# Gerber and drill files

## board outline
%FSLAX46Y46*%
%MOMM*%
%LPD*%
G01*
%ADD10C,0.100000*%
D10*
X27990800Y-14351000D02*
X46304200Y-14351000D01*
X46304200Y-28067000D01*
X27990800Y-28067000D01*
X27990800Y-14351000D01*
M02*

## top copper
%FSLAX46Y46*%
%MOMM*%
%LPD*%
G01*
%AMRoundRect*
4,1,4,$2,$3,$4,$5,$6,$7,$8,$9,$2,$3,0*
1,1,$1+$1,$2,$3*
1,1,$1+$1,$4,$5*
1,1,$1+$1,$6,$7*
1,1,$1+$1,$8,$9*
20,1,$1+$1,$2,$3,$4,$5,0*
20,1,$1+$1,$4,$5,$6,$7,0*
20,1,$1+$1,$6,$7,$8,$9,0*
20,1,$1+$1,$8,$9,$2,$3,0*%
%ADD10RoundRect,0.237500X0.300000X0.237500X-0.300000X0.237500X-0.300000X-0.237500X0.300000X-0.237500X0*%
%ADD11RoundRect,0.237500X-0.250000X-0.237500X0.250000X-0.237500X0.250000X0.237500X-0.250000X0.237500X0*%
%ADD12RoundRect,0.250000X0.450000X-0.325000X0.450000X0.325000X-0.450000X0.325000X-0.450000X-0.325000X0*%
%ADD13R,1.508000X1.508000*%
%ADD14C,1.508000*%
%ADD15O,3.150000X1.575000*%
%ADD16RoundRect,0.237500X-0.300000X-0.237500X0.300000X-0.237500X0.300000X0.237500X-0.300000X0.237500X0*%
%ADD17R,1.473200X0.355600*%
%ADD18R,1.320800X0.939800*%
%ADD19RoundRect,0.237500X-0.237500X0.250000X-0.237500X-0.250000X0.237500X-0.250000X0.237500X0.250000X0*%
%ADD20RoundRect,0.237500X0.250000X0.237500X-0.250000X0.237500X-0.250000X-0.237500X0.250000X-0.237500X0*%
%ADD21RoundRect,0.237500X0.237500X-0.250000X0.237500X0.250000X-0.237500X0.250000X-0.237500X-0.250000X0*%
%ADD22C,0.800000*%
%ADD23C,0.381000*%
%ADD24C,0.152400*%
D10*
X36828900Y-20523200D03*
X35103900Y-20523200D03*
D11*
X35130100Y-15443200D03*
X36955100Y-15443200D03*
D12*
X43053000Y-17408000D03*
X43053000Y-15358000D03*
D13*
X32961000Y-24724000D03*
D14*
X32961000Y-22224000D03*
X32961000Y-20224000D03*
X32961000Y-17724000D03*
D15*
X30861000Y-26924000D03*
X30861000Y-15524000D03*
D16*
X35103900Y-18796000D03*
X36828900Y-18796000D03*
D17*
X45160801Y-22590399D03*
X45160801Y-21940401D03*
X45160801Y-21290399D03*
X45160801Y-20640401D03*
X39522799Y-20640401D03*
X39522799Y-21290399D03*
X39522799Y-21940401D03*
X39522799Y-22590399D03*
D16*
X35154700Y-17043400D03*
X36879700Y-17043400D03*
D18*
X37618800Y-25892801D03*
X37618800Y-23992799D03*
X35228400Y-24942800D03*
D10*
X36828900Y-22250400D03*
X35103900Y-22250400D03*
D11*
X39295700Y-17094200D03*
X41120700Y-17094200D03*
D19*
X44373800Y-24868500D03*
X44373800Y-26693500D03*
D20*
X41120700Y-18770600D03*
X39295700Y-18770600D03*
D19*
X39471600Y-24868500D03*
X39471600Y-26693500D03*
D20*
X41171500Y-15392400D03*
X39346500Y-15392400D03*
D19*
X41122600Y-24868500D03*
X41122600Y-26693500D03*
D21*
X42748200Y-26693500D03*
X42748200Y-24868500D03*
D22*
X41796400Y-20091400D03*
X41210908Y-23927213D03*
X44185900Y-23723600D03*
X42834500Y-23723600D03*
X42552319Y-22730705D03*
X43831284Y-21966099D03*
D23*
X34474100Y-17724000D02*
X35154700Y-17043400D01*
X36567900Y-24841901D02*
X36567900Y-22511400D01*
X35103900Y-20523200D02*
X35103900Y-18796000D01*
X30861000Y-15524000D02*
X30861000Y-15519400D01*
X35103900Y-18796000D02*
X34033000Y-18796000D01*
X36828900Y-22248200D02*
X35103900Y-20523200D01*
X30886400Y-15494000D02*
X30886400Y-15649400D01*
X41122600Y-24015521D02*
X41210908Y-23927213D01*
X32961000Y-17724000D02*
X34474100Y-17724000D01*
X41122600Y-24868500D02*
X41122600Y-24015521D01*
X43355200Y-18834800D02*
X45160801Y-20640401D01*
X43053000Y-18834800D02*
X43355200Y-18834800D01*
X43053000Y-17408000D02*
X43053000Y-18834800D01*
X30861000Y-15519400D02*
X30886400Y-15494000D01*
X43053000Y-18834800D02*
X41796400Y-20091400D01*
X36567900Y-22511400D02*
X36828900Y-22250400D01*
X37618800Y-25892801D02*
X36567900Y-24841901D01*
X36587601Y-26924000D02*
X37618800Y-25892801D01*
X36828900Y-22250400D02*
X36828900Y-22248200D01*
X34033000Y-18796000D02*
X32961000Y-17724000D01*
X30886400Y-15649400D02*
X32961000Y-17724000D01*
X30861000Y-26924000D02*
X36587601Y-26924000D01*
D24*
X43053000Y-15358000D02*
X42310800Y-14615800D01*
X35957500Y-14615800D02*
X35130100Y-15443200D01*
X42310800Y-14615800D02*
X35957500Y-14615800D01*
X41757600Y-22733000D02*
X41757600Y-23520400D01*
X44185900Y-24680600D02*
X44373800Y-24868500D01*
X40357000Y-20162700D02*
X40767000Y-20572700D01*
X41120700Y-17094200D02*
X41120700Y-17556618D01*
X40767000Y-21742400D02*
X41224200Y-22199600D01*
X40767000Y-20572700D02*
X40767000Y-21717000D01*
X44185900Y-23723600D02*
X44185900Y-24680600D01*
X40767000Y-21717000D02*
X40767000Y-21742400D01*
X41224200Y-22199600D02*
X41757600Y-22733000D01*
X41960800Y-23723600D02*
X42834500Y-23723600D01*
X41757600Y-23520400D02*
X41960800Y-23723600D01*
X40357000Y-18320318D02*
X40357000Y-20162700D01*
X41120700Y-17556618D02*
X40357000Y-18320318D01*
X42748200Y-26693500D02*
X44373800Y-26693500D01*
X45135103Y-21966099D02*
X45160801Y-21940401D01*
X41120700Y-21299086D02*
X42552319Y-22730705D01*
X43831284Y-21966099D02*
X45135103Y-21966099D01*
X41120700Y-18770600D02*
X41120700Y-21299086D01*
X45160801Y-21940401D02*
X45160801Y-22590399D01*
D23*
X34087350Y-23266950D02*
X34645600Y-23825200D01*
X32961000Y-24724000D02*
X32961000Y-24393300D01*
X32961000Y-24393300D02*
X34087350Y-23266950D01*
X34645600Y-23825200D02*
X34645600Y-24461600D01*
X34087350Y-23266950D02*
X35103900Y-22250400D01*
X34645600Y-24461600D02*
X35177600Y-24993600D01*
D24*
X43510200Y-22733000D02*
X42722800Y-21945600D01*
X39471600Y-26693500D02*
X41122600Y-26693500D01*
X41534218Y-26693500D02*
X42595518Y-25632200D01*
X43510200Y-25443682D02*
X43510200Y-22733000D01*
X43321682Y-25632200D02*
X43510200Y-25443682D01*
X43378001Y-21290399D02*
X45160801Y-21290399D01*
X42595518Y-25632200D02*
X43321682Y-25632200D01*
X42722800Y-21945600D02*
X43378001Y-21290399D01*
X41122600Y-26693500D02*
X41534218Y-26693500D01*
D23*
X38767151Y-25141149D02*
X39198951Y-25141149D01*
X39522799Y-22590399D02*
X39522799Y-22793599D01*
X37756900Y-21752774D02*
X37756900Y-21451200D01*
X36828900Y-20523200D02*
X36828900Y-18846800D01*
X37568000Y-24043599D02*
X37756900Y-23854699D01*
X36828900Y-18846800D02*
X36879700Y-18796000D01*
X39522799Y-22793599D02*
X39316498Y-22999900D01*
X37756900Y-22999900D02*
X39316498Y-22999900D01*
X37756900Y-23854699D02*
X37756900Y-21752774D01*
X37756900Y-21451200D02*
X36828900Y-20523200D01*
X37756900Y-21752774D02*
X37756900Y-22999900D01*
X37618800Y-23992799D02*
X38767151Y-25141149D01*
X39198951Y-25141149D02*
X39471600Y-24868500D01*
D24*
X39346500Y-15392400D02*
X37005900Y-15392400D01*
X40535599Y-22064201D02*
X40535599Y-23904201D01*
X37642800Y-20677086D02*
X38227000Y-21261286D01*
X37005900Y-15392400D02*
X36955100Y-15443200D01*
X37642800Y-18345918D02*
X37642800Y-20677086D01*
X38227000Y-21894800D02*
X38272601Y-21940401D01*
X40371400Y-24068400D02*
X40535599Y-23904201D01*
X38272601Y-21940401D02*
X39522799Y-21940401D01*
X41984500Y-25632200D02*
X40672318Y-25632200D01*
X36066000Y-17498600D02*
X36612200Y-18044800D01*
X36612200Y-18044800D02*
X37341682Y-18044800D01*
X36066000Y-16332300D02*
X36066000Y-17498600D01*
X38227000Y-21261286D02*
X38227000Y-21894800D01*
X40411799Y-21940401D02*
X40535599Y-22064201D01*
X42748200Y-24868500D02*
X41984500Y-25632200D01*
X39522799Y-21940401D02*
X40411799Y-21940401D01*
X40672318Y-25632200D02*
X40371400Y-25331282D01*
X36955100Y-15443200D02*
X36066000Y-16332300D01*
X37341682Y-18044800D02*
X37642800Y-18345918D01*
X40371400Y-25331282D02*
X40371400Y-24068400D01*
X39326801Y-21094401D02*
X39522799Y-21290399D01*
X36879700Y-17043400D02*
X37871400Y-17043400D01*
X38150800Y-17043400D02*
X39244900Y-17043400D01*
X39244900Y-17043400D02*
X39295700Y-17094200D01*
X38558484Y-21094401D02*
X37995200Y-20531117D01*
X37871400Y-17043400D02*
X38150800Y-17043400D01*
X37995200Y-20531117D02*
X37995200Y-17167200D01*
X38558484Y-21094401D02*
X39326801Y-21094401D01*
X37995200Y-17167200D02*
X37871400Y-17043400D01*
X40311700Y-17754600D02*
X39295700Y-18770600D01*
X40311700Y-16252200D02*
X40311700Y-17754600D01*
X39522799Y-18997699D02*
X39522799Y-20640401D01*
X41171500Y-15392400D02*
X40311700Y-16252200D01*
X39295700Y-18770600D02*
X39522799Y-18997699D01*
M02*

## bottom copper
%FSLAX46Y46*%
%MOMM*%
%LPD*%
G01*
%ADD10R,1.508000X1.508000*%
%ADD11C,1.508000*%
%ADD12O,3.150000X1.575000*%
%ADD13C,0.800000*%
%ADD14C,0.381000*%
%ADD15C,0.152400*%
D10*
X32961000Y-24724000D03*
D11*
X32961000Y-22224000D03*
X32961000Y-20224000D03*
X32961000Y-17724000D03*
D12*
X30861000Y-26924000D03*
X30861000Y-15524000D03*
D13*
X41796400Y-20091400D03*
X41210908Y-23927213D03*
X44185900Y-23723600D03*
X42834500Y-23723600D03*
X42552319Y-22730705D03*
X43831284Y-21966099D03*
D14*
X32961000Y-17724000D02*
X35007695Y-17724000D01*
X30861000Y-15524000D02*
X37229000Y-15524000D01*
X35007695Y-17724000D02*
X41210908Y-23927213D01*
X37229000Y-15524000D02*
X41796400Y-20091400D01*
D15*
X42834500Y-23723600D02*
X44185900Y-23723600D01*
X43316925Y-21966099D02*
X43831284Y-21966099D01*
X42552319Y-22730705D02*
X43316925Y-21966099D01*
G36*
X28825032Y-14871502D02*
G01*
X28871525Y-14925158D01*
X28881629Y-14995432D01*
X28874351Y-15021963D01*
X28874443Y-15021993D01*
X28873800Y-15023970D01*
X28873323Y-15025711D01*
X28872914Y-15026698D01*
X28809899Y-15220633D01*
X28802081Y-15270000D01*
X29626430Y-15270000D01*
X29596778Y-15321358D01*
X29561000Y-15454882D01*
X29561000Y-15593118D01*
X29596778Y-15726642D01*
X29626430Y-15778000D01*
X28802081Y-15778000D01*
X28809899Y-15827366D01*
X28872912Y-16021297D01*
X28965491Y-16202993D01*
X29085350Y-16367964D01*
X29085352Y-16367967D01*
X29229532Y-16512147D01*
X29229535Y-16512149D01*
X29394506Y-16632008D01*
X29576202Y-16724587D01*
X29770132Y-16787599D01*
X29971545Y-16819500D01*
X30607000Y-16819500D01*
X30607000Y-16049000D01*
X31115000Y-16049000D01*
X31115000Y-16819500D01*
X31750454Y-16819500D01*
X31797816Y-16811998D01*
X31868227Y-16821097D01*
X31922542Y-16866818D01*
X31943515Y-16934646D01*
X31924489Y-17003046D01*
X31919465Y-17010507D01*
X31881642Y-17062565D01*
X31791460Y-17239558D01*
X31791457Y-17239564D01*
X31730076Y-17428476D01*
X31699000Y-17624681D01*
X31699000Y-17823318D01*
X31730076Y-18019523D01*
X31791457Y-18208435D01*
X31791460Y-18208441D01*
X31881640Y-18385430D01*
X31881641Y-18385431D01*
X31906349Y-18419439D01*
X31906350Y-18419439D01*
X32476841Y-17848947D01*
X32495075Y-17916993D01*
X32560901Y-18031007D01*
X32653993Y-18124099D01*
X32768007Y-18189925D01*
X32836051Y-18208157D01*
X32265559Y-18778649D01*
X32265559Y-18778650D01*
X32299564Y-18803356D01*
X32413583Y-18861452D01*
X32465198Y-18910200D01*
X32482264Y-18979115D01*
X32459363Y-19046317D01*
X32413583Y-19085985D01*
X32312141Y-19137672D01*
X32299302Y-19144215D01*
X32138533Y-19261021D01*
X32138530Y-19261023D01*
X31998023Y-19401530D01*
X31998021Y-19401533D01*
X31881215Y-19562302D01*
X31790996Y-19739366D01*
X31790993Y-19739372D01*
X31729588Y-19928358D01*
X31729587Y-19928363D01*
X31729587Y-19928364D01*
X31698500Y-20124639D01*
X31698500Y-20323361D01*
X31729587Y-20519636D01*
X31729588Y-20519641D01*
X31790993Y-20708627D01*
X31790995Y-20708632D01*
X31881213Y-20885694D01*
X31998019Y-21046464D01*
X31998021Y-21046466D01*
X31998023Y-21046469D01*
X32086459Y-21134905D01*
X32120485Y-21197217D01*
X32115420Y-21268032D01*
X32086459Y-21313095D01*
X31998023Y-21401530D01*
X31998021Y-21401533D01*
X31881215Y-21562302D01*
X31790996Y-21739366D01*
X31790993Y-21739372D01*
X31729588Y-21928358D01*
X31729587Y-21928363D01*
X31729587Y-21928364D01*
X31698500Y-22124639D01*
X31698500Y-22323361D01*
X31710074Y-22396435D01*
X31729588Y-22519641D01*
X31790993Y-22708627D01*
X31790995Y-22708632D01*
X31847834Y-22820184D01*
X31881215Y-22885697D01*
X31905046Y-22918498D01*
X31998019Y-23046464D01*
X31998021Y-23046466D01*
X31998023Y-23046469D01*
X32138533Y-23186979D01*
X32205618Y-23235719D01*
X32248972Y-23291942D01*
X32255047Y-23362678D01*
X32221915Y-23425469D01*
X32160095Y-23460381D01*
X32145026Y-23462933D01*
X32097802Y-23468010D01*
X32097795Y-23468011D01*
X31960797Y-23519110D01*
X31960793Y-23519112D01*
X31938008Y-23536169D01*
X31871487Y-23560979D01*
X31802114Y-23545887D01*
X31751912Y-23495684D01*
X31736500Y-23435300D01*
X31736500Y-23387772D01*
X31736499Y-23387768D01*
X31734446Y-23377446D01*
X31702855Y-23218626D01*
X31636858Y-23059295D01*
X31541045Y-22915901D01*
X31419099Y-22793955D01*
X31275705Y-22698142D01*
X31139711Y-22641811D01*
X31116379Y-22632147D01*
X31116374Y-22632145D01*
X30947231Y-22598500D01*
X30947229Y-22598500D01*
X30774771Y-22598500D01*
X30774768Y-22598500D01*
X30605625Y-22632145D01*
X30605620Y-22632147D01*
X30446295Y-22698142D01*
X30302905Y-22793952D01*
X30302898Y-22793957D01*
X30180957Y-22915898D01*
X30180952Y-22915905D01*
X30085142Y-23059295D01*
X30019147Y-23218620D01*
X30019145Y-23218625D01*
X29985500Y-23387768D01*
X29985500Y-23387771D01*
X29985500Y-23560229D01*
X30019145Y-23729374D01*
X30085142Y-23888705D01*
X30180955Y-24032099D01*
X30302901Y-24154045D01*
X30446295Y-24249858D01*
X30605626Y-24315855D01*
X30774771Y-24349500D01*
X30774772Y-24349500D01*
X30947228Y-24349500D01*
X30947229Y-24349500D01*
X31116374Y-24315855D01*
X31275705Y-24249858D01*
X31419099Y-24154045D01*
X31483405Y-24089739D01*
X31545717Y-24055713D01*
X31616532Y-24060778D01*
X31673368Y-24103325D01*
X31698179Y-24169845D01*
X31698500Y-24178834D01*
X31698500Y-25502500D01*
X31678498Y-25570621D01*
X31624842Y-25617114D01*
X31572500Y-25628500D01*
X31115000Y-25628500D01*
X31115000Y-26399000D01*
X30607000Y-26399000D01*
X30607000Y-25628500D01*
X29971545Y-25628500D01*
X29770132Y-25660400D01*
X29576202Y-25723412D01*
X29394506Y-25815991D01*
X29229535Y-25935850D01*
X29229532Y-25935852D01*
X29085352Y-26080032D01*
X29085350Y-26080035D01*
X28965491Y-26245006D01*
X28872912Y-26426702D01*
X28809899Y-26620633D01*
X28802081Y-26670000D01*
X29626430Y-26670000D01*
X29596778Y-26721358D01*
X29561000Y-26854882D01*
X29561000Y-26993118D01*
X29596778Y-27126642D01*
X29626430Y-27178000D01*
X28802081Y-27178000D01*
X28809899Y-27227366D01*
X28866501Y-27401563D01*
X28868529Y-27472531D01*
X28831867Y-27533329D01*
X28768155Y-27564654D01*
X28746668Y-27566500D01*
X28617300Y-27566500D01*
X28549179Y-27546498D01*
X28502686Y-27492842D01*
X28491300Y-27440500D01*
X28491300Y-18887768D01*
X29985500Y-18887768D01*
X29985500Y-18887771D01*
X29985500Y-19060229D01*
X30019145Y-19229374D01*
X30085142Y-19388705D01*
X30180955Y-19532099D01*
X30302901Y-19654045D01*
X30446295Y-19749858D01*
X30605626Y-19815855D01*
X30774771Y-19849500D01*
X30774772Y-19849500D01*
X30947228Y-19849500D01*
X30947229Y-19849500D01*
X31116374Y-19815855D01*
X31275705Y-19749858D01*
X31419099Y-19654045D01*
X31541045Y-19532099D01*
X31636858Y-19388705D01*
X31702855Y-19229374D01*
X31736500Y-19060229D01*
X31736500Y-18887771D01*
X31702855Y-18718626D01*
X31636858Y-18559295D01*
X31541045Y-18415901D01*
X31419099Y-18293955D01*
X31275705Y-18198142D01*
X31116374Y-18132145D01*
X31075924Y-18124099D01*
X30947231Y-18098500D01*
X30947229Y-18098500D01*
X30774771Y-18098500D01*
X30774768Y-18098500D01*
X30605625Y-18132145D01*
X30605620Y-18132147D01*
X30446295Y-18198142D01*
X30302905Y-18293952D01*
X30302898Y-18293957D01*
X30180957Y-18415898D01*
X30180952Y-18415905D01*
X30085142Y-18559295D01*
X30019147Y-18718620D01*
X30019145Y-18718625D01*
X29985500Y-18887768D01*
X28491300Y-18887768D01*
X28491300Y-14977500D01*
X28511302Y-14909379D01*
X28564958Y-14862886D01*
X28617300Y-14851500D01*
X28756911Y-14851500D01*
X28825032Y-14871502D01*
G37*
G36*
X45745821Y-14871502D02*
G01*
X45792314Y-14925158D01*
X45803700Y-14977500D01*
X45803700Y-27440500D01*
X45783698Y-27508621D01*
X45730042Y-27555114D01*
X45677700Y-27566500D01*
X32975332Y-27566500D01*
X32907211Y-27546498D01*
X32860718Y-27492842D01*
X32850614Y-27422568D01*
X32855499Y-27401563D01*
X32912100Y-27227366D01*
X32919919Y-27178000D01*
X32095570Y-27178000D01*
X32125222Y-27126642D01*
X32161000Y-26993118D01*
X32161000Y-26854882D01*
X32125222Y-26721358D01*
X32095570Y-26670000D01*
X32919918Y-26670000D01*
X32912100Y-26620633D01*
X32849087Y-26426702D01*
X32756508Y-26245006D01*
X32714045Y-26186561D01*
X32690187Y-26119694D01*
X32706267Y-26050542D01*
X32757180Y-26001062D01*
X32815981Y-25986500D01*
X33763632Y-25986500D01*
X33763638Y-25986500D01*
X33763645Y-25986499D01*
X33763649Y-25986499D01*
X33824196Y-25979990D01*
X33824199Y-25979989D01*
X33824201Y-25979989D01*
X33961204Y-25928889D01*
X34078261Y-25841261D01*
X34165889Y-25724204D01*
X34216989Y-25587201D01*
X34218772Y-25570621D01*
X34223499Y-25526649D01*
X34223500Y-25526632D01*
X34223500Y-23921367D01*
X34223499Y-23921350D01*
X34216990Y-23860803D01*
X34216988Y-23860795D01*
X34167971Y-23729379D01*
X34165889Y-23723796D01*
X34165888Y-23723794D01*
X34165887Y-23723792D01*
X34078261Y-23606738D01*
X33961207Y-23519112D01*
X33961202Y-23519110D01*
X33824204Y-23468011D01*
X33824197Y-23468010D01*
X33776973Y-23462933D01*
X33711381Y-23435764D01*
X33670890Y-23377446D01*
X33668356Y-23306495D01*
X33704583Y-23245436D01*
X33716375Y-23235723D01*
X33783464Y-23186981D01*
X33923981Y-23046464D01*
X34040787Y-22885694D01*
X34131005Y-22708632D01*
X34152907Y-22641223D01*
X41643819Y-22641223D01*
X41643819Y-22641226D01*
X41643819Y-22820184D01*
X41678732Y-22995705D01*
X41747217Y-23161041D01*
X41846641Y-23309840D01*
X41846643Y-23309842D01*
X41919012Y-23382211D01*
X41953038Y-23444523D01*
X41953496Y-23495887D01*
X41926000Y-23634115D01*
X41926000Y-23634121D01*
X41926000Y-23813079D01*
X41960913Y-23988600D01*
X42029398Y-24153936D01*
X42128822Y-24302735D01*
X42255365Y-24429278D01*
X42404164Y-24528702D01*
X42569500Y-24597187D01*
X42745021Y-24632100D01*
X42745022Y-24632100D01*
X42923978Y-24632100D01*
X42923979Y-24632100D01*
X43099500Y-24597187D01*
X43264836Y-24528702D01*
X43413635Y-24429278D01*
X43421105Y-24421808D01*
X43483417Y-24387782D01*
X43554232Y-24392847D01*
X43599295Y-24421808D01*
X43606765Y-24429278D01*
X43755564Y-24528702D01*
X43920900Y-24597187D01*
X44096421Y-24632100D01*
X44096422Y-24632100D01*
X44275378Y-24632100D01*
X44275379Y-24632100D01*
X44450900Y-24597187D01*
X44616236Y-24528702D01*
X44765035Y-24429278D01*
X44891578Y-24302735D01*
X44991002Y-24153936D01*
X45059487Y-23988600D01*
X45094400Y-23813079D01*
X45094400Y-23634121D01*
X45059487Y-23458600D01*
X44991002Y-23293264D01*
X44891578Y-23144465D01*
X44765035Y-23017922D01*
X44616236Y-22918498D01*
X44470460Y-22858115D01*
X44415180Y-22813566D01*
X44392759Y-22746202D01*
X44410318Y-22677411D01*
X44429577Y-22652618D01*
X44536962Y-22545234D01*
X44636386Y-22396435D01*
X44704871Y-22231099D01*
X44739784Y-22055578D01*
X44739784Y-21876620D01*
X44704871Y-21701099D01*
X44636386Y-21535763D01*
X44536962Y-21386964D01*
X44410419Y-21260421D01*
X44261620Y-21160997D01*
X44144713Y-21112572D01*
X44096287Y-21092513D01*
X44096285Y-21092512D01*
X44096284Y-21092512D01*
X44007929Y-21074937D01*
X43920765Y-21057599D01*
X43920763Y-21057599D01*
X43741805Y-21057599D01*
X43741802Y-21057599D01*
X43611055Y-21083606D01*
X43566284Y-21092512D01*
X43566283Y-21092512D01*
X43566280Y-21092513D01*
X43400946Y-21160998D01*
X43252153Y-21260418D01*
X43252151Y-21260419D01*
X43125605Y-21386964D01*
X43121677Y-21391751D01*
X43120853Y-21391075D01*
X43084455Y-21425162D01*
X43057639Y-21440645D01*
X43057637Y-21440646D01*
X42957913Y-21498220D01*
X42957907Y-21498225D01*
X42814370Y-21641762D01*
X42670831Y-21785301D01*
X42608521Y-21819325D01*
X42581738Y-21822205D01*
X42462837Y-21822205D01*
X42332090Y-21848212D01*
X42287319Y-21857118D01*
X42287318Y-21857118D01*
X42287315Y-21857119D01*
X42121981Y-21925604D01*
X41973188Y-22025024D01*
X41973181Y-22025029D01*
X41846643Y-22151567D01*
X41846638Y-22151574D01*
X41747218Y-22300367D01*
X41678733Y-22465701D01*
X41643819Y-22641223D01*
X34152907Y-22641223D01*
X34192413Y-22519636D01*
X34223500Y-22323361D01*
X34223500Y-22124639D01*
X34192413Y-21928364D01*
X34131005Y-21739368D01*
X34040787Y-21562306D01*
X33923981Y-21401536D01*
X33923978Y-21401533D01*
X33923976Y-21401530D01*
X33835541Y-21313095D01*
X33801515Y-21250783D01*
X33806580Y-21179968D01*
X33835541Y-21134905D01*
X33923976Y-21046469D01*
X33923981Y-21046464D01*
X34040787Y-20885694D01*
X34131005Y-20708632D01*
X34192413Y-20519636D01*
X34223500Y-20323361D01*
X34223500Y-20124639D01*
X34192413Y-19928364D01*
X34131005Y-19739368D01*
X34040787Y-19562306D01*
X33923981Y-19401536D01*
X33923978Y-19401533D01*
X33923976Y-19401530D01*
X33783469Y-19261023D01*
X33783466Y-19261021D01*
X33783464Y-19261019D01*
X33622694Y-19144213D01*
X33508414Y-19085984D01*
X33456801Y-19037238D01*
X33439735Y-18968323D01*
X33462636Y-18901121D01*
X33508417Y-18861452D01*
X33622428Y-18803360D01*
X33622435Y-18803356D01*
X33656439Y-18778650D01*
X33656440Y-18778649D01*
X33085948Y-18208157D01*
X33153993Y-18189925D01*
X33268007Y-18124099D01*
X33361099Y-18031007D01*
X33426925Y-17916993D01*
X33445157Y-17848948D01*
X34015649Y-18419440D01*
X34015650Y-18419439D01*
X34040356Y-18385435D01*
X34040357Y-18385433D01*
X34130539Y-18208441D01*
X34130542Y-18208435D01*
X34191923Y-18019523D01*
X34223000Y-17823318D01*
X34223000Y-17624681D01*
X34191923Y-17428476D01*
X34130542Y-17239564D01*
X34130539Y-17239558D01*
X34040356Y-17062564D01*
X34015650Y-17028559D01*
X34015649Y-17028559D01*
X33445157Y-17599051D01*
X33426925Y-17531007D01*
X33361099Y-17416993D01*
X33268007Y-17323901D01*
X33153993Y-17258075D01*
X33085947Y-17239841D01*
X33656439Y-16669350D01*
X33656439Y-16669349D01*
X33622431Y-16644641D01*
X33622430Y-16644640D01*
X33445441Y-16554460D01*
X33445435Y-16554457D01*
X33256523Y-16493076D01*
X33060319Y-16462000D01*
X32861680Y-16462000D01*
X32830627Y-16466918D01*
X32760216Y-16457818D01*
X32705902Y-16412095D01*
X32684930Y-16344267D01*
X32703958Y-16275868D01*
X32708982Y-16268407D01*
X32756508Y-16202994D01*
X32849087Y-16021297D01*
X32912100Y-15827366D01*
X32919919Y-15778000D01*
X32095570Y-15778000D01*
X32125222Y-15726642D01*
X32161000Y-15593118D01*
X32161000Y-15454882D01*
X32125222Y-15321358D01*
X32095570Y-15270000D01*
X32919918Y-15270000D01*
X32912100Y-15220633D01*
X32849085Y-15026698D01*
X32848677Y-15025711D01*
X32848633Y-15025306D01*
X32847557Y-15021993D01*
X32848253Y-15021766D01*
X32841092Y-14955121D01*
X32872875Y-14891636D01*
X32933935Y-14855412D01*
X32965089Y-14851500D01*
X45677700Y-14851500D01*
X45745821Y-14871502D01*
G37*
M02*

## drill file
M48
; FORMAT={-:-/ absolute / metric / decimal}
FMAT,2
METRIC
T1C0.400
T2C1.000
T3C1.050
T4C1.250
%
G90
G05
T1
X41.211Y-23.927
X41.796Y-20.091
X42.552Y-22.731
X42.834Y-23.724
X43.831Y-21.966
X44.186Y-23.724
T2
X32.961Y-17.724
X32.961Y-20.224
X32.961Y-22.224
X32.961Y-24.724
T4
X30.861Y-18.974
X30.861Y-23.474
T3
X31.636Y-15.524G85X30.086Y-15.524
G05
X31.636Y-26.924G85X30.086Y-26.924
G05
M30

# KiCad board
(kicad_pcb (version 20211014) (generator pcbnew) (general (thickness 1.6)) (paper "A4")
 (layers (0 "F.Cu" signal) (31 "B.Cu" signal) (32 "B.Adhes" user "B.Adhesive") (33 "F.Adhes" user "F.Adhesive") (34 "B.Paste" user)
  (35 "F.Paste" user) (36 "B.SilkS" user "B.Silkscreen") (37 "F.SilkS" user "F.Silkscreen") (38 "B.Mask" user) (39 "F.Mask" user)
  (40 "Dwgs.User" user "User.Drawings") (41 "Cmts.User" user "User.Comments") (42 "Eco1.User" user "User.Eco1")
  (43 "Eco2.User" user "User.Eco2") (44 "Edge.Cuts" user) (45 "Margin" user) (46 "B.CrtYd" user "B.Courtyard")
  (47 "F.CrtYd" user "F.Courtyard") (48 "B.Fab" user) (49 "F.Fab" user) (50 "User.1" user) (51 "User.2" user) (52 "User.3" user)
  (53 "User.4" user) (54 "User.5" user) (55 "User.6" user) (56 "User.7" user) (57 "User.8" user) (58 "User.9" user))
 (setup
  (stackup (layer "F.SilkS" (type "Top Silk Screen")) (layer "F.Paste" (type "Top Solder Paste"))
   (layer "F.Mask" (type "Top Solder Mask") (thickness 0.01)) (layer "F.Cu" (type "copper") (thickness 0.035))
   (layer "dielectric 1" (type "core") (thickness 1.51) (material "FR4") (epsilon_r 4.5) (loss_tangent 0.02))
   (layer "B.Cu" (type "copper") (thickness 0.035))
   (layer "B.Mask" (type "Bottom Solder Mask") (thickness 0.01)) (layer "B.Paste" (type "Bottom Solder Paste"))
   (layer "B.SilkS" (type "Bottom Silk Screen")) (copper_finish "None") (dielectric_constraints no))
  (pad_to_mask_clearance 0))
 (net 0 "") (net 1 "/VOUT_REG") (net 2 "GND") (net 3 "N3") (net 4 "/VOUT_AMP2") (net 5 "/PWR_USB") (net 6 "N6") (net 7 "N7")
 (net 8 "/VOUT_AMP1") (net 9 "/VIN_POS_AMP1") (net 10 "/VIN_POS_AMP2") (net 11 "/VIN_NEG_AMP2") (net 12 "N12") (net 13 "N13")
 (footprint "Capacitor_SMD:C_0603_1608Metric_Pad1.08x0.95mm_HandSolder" (layer "F.Cu") (at 35.9664 20.5232 180)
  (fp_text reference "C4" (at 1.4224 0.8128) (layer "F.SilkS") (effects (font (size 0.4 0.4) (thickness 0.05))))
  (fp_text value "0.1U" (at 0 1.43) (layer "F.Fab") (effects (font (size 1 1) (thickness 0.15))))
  (pad "1" smd roundrect (at -0.8625 0 180) (size 1.075 0.95) (layers "F.Cu" "F.Paste" "F.Mask") (roundrect_rratio 0.25) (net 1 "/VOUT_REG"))
  (pad "2" smd roundrect (at 0.8625 0 180) (size 1.075 0.95) (layers "F.Cu" "F.Paste" "F.Mask") (roundrect_rratio 0.25) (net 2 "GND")))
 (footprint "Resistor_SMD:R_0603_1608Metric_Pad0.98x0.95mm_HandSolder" (layer "F.Cu") (at 36.0426 15.4432)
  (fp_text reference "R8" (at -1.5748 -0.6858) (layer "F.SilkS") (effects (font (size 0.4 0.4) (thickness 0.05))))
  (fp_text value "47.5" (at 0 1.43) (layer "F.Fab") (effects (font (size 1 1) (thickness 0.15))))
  (pad "1" smd roundrect (at -0.9125 0) (size 0.975 0.95) (layers "F.Cu" "F.Paste" "F.Mask") (roundrect_rratio 0.25) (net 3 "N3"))
  (pad "2" smd roundrect (at 0.9125 0) (size 0.975 0.95) (layers "F.Cu" "F.Paste" "F.Mask") (roundrect_rratio 0.25) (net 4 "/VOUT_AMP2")))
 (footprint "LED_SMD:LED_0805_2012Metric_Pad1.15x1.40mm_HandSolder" (layer "F.Cu") (at 43.053 16.383 90)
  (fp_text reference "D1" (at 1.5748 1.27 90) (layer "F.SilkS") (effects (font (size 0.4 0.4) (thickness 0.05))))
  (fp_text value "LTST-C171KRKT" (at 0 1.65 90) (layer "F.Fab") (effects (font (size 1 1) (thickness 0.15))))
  (pad "1" smd roundrect (at -1.025 0 90) (size 1.15 1.4) (layers "F.Cu" "F.Paste" "F.Mask") (roundrect_rratio 0.217391) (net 2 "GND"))
  (pad "2" smd roundrect (at 1.025 0 90) (size 1.15 1.4) (layers "F.Cu" "F.Paste" "F.Mask") (roundrect_rratio 0.217391) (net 3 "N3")))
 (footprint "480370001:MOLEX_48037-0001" (layer "F.Cu") (at 30.861 21.224 -90)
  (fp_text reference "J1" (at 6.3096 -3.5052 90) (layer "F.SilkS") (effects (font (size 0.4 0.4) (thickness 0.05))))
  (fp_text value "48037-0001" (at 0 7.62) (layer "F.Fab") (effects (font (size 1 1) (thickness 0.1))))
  (pad "" np_thru_hole circle (at -2.25 0 270) (size 1.25 1.25) (drill 1.25) (layers *.Cu *.Mask))
  (pad "" np_thru_hole circle (at 2.25 0 270) (size 1.25 1.25) (drill 1.25) (layers *.Cu *.Mask))
  (pad "1" thru_hole rect (at 3.5 -2.1 270) (size 1.508 1.508) (drill 1) (layers *.Cu *.Mask) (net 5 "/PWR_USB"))
  (pad "2" thru_hole circle (at 1 -2.1 270) (size 1.508 1.508) (drill 1) (layers *.Cu *.Mask) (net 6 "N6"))
  (pad "3" thru_hole circle (at -1 -2.1 270) (size 1.508 1.508) (drill 1) (layers *.Cu *.Mask) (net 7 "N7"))
  (pad "4" thru_hole circle (at -3.5 -2.1 270) (size 1.508 1.508) (drill 1) (layers *.Cu *.Mask) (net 2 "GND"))
  (pad "S1" thru_hole oval (at 5.7 0 270) (size 1.575 3.15) (drill oval 1.05 2.6) (layers *.Cu *.Mask) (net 2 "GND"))
  (pad "S2" thru_hole oval (at -5.7 0 270) (size 1.575 3.15) (drill oval 1.05 2.6) (layers *.Cu *.Mask) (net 2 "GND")))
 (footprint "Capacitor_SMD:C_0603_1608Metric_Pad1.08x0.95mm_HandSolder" (layer "F.Cu") (at 35.9664 18.796)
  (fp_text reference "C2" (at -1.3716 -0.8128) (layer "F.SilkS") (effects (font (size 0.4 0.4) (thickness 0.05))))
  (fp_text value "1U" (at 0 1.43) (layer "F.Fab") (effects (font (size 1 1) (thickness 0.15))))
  (pad "1" smd roundrect (at -0.8625 0) (size 1.075 0.95) (layers "F.Cu" "F.Paste" "F.Mask") (roundrect_rratio 0.25) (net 2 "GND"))
  (pad "2" smd roundrect (at 0.8625 0) (size 1.075 0.95) (layers "F.Cu" "F.Paste" "F.Mask") (roundrect_rratio 0.25) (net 1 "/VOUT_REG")))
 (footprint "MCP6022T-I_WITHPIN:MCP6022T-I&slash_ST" (layer "F.Cu") (at 42.3418 21.6154 180)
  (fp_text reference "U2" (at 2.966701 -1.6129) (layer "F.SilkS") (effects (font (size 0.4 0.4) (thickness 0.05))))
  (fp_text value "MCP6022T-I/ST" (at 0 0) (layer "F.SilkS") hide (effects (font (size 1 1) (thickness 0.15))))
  (pad "1" smd rect (at -2.819001 -0.974999 180) (size 1.4732 0.3556) (layers "F.Cu" "F.Paste" "F.Mask") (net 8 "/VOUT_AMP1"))
  (pad "2" smd rect (at -2.819001 -0.325001 180) (size 1.4732 0.3556) (layers "F.Cu" "F.Paste" "F.Mask") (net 8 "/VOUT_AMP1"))
  (pad "3" smd rect (at -2.819001 0.325001 180) (size 1.4732 0.3556) (layers "F.Cu" "F.Paste" "F.Mask") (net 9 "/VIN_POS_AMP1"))
  (pad "4" smd rect (at -2.819001 0.974999 180) (size 1.4732 0.3556) (layers "F.Cu" "F.Paste" "F.Mask") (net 2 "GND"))
  (pad "5" smd rect (at 2.819001 0.974999 180) (size 1.4732 0.3556) (layers "F.Cu" "F.Paste" "F.Mask") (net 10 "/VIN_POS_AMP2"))
  (pad "6" smd rect (at 2.819001 0.325001 180) (size 1.4732 0.3556) (layers "F.Cu" "F.Paste" "F.Mask") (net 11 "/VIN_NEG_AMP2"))
  (pad "7" smd rect (at 2.819001 -0.325001 180) (size 1.4732 0.3556) (layers "F.Cu" "F.Paste" "F.Mask") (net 4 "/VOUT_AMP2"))
  (pad "8" smd rect (at 2.819001 -0.974999 180) (size 1.4732 0.3556) (layers "F.Cu" "F.Paste" "F.Mask") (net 1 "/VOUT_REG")))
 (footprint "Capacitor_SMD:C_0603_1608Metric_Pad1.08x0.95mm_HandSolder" (layer "F.Cu") (at 36.0172 17.0434)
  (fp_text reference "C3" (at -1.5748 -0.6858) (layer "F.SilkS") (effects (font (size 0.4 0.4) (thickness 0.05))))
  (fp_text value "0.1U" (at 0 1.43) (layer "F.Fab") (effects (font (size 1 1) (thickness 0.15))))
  (pad "1" smd roundrect (at -0.8625 0) (size 1.075 0.95) (layers "F.Cu" "F.Paste" "F.Mask") (roundrect_rratio 0.25) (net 2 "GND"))
  (pad "2" smd roundrect (at 0.8625 0) (size 1.075 0.95) (layers "F.Cu" "F.Paste" "F.Mask") (roundrect_rratio 0.25) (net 11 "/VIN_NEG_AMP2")))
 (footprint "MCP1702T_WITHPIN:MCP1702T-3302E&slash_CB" (layer "F.Cu") (at 36.4236 24.9428 90)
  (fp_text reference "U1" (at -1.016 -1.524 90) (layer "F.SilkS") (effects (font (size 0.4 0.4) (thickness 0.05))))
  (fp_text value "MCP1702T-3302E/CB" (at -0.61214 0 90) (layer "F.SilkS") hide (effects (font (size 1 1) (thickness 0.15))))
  (pad "1" smd rect (at -0.950001 1.1952 90) (size 0.9398 1.3208) (layers "F.Cu" "F.Paste" "F.Mask") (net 2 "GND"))
  (pad "2" smd rect (at 0.950001 1.1952 90) (size 0.9398 1.3208) (layers "F.Cu" "F.Paste" "F.Mask") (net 1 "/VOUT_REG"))
  (pad "3" smd rect (at 0 -1.1952 90) (size 0.9398 1.3208) (layers "F.Cu" "F.Paste" "F.Mask") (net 5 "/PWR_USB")))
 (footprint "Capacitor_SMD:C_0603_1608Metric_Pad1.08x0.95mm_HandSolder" (layer "F.Cu") (at 35.9664 22.2504 180)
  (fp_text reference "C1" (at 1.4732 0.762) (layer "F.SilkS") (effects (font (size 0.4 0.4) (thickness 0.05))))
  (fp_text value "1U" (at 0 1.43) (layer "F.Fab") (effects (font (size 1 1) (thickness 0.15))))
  (pad "1" smd roundrect (at -0.8625 0 180) (size 1.075 0.95) (layers "F.Cu" "F.Paste" "F.Mask") (roundrect_rratio 0.25) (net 2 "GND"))
  (pad "2" smd roundrect (at 0.8625 0 180) (size 1.075 0.95) (layers "F.Cu" "F.Paste" "F.Mask") (roundrect_rratio 0.25) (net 5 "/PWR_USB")))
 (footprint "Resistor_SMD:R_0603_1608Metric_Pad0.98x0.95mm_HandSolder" (layer "F.Cu") (at 40.2082 17.0942)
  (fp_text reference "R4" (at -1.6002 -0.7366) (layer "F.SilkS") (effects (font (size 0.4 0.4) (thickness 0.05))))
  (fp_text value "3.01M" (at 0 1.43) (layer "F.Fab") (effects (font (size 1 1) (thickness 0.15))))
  (pad "1" smd roundrect (at -0.9125 0) (size 0.975 0.95) (layers "F.Cu" "F.Paste" "F.Mask") (roundrect_rratio 0.25)
   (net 11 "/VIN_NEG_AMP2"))
  (pad "2" smd roundrect (at 0.9125 0) (size 0.975 0.95) (layers "F.Cu" "F.Paste" "F.Mask") (roundrect_rratio 0.25) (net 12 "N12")))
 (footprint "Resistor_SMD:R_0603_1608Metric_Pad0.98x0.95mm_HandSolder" (layer "F.Cu") (at 44.3738 25.781 -90)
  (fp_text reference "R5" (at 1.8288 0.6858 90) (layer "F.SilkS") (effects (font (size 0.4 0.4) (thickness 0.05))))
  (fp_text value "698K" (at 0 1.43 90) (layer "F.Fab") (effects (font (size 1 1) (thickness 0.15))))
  (pad "1" smd roundrect (at -0.9125 0 270) (size 0.975 0.95) (layers "F.Cu" "F.Paste" "F.Mask") (roundrect_rratio 0.25) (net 12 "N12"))
  (pad "2" smd roundrect (at 0.9125 0 270) (size 0.975 0.95) (layers "F.Cu" "F.Paste" "F.Mask") (roundrect_rratio 0.25) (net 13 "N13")))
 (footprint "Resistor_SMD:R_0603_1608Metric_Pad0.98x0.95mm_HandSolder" (layer "F.Cu") (at 40.2082 18.7706 180)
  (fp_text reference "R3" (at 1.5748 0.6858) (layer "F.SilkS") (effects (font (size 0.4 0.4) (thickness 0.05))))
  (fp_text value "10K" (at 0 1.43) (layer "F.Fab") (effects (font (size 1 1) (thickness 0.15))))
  (pad "1" smd roundrect (at -0.9125 0 180) (size 0.975 0.95) (layers "F.Cu" "F.Paste" "F.Mask") (roundrect_rratio 0.25)
   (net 8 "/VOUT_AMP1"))
  (pad "2" smd roundrect (at 0.9125 0 180) (size 0.975 0.95) (layers "F.Cu" "F.Paste" "F.Mask") (roundrect_rratio 0.25)
   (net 10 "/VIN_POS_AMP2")))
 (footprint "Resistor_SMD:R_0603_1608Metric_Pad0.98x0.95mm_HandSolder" (layer "F.Cu") (at 39.4716 25.781 -90)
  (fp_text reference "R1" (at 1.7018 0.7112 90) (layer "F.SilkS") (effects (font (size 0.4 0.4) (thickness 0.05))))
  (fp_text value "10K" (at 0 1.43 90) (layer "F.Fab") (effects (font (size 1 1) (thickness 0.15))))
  (pad "1" smd roundrect (at -0.9125 0 270) (size 0.975 0.95) (layers "F.Cu" "F.Paste" "F.Mask") (roundrect_rratio 0.25) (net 1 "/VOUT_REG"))
  (pad "2" smd roundrect (at 0.9125 0 270) (size 0.975 0.95) (layers "F.Cu" "F.Paste" "F.Mask") (roundrect_rratio 0.25)
   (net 9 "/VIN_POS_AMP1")))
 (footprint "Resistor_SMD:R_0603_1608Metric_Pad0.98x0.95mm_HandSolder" (layer "F.Cu") (at 40.259 15.3924 180)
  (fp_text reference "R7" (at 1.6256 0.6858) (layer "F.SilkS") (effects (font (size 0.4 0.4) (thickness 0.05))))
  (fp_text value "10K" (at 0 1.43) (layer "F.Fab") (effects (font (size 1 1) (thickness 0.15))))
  (pad "1" smd roundrect (at -0.9125 0 180) (size 0.975 0.95) (layers "F.Cu" "F.Paste" "F.Mask") (roundrect_rratio 0.25)
   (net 10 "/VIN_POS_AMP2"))
  (pad "2" smd roundrect (at 0.9125 0 180) (size 0.975 0.95) (layers "F.Cu" "F.Paste" "F.Mask") (roundrect_rratio 0.25) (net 4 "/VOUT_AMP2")))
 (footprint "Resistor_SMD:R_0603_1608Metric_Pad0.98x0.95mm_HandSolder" (layer "F.Cu") (at 41.1226 25.781 -90)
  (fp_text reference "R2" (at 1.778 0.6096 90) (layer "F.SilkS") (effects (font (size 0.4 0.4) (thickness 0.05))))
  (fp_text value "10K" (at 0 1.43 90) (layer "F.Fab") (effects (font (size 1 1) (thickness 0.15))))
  (pad "1" smd roundrect (at -0.9125 0 270) (size 0.975 0.95) (layers "F.Cu" "F.Paste" "F.Mask") (roundrect_rratio 0.25) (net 2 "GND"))
  (pad "2" smd roundrect (at 0.9125 0 270) (size 0.975 0.95) (layers "F.Cu" "F.Paste" "F.Mask") (roundrect_rratio 0.25)
   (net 9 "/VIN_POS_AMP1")))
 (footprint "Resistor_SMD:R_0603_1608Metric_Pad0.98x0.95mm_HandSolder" (layer "F.Cu") (at 42.7482 25.781 90)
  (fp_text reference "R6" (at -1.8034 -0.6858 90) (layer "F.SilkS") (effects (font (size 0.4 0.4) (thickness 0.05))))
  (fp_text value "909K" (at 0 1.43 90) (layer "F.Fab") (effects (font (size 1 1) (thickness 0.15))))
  (pad "1" smd roundrect (at -0.9125 0 90) (size 0.975 0.95) (layers "F.Cu" "F.Paste" "F.Mask") (roundrect_rratio 0.25) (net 13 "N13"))
  (pad "2" smd roundrect (at 0.9125 0 90) (size 0.975 0.95) (layers "F.Cu" "F.Paste" "F.Mask") (roundrect_rratio 0.25) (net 4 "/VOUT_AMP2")))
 (gr_rect (start 46.3042 28.067) (end 27.9908 14.351) (layer "Edge.Cuts") (width 0.1) (fill none))
 (segment (start 34.4741 17.724) (end 35.1547 17.0434) (width 0.381) (layer "F.Cu") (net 2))
 (segment (start 36.5679 24.841901) (end 36.5679 22.5114) (width 0.381) (layer "F.Cu") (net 2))
 (segment (start 35.1039 20.5232) (end 35.1039 18.796) (width 0.381) (layer "F.Cu") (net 2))
 (segment (start 30.861 15.524) (end 30.861 15.5194) (width 0.381) (layer "F.Cu") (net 2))
 (segment (start 35.1039 18.796) (end 34.033 18.796) (width 0.381) (layer "F.Cu") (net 2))
 (segment (start 36.8289 22.2482) (end 35.1039 20.5232) (width 0.381) (layer "F.Cu") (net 2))
 (segment (start 30.8864 15.494) (end 30.8864 15.6494) (width 0.381) (layer "F.Cu") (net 2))
 (segment (start 41.1226 24.015521) (end 41.210908 23.927213) (width 0.381) (layer "F.Cu") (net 2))
 (segment (start 32.961 17.724) (end 34.4741 17.724) (width 0.381) (layer "F.Cu") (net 2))
 (segment (start 41.1226 24.8685) (end 41.1226 24.015521) (width 0.381) (layer "F.Cu") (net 2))
 (segment (start 43.3552 18.8348) (end 45.160801 20.640401) (width 0.381) (layer "F.Cu") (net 2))
 (segment (start 43.053 18.8348) (end 43.3552 18.8348) (width 0.381) (layer "F.Cu") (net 2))
 (segment (start 43.053 17.408) (end 43.053 18.8348) (width 0.381) (layer "F.Cu") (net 2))
 (segment (start 30.861 15.5194) (end 30.8864 15.494) (width 0.381) (layer "F.Cu") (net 2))
 (segment (start 43.053 18.8348) (end 41.7964 20.0914) (width 0.381) (layer "F.Cu") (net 2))
 (segment (start 36.5679 22.5114) (end 36.8289 22.2504) (width 0.381) (layer "F.Cu") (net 2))
 (segment (start 37.6188 25.892801) (end 36.5679 24.841901) (width 0.381) (layer "F.Cu") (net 2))
 (segment (start 36.587601 26.924) (end 37.6188 25.892801) (width 0.381) (layer "F.Cu") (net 2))
 (segment (start 36.8289 22.2504) (end 36.8289 22.2482) (width 0.381) (layer "F.Cu") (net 2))
 (segment (start 34.033 18.796) (end 32.961 17.724) (width 0.381) (layer "F.Cu") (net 2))
 (segment (start 30.8864 15.6494) (end 32.961 17.724) (width 0.381) (layer "F.Cu") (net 2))
 (segment (start 30.861 26.924) (end 36.587601 26.924) (width 0.381) (layer "F.Cu") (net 2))
 (via (at 41.7964 20.0914) (size 0.8) (drill 0.4) (layers "F.Cu" "B.Cu") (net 2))
 (via (at 41.210908 23.927213) (size 0.8) (drill 0.4) (layers "F.Cu" "B.Cu") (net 2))
 (segment (start 32.961 17.724) (end 35.007695 17.724) (width 0.381) (layer "B.Cu") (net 2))
 (segment (start 30.861 15.524) (end 37.229 15.524) (width 0.381) (layer "B.Cu") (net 2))
 (segment (start 35.007695 17.724) (end 41.210908 23.927213) (width 0.381) (layer "B.Cu") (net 2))
 (segment (start 37.229 15.524) (end 41.7964 20.0914) (width 0.381) (layer "B.Cu") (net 2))
 (segment (start 43.053 15.358) (end 42.3108 14.6158) (width 0.1524) (layer "F.Cu") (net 3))
 (segment (start 35.9575 14.6158) (end 35.1301 15.4432) (width 0.1524) (layer "F.Cu") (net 3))
 (segment (start 42.3108 14.6158) (end 35.9575 14.6158) (width 0.1524) (layer "F.Cu") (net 3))
 (segment (start 41.7576 22.733) (end 41.7576 23.5204) (width 0.1524) (layer "F.Cu") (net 12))
 (segment (start 44.1859 24.6806) (end 44.3738 24.8685) (width 0.1524) (layer "F.Cu") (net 12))
 (segment (start 40.357 20.1627) (end 40.767 20.5727) (width 0.1524) (layer "F.Cu") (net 12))
 (segment (start 41.1207 17.0942) (end 41.1207 17.556618) (width 0.1524) (layer "F.Cu") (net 12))
 (segment (start 40.767 21.7424) (end 41.2242 22.1996) (width 0.1524) (layer "F.Cu") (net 12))
 (segment (start 40.767 20.5727) (end 40.767 21.717) (width 0.1524) (layer "F.Cu") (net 12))
 (segment (start 44.1859 23.7236) (end 44.1859 24.6806) (width 0.1524) (layer "F.Cu") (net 12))
 (segment (start 40.767 21.717) (end 40.767 21.7424) (width 0.1524) (layer "F.Cu") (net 12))
 (segment (start 41.2242 22.1996) (end 41.7576 22.733) (width 0.1524) (layer "F.Cu") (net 12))
 (segment (start 41.9608 23.7236) (end 42.8345 23.7236) (width 0.1524) (layer "F.Cu") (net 12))
 (segment (start 41.7576 23.5204) (end 41.9608 23.7236) (width 0.1524) (layer "F.Cu") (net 12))
 (segment (start 40.357 18.320318) (end 40.357 20.1627) (width 0.1524) (layer "F.Cu") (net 12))
 (segment (start 41.1207 17.556618) (end 40.357 18.320318) (width 0.1524) (layer "F.Cu") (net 12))
 (via (at 44.1859 23.7236) (size 0.8) (drill 0.4) (layers "F.Cu" "B.Cu") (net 12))
 (via (at 42.8345 23.7236) (size 0.8) (drill 0.4) (layers "F.Cu" "B.Cu") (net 12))
 (segment (start 42.8345 23.7236) (end 44.1859 23.7236) (width 0.1524) (layer "B.Cu") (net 12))
 (segment (start 42.7482 26.6935) (end 44.3738 26.6935) (width 0.1524) (layer "F.Cu") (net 13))
 (segment (start 45.135103 21.966099) (end 45.160801 21.940401) (width 0.1524) (layer "F.Cu") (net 8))
 (segment (start 41.1207 21.299086) (end 42.552319 22.730705) (width 0.1524) (layer "F.Cu") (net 8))
 (segment (start 43.831284 21.966099) (end 45.135103 21.966099) (width 0.1524) (layer "F.Cu") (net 8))
 (segment (start 41.1207 18.7706) (end 41.1207 21.299086) (width 0.1524) (layer "F.Cu") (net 8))
 (segment (start 45.160801 21.940401) (end 45.160801 22.590399) (width 0.1524) (layer "F.Cu") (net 8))
 (via (at 42.552319 22.730705) (size 0.8) (drill 0.4) (layers "F.Cu" "B.Cu") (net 8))
 (via (at 43.831284 21.966099) (size 0.8) (drill 0.4) (layers "F.Cu" "B.Cu") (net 8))
 (segment (start 43.316925 21.966099) (end 43.831284 21.966099) (width 0.1524) (layer "B.Cu") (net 8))
 (segment (start 42.552319 22.730705) (end 43.316925 21.966099) (width 0.1524) (layer "B.Cu") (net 8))
 (segment (start 34.08735 23.26695) (end 34.6456 23.8252) (width 0.381) (layer "F.Cu") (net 5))
 (segment (start 32.961 24.724) (end 32.961 24.3933) (width 0.381) (layer "F.Cu") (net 5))
 (segment (start 32.961 24.3933) (end 34.08735 23.26695) (width 0.381) (layer "F.Cu") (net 5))
 (segment (start 34.6456 23.8252) (end 34.6456 24.4616) (width 0.381) (layer "F.Cu") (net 5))
 (segment (start 34.08735 23.26695) (end 35.1039 22.2504) (width 0.381) (layer "F.Cu") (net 5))
 (segment (start 34.6456 24.4616) (end 35.1776 24.9936) (width 0.381) (layer "F.Cu") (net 5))
 (segment (start 43.5102 22.733) (end 42.7228 21.9456) (width 0.1524) (layer "F.Cu") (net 9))
 (segment (start 39.4716 26.6935) (end 41.1226 26.6935) (width 0.1524) (layer "F.Cu") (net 9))
 (segment (start 41.534218 26.6935) (end 42.595518 25.6322) (width 0.1524) (layer "F.Cu") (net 9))
 (segment (start 43.5102 25.443682) (end 43.5102 22.733) (width 0.1524) (layer "F.Cu") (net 9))
 (segment (start 43.321682 25.6322) (end 43.5102 25.443682) (width 0.1524) (layer "F.Cu") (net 9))
 (segment (start 43.378001 21.290399) (end 45.160801 21.290399) (width 0.1524) (layer "F.Cu") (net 9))
 (segment (start 42.595518 25.6322) (end 43.321682 25.6322) (width 0.1524) (layer "F.Cu") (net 9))
 (segment (start 42.7228 21.9456) (end 43.378001 21.290399) (width 0.1524) (layer "F.Cu") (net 9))
 (segment (start 41.1226 26.6935) (end 41.534218 26.6935) (width 0.1524) (layer "F.Cu") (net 9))
 (segment (start 38.767151 25.141149) (end 39.198951 25.141149) (width 0.381) (layer "F.Cu") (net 1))
 (segment (start 39.522799 22.590399) (end 39.522799 22.793599) (width 0.381) (layer "F.Cu") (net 1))
 (segment (start 37.7569 21.752774) (end 37.7569 21.4512) (width 0.381) (layer "F.Cu") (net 1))
 (segment (start 36.8289 20.5232) (end 36.8289 18.8468) (width 0.381) (layer "F.Cu") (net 1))
 (segment (start 37.568 24.043599) (end 37.7569 23.854699) (width 0.381) (layer "F.Cu") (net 1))
 (segment (start 36.8289 18.8468) (end 36.8797 18.796) (width 0.381) (layer "F.Cu") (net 1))
 (segment (start 39.522799 22.793599) (end 39.316498 22.9999) (width 0.381) (layer "F.Cu") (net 1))
 (segment (start 37.7569 22.9999) (end 39.316498 22.9999) (width 0.381) (layer "F.Cu") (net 1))
 (segment (start 37.7569 23.854699) (end 37.7569 21.752774) (width 0.381) (layer "F.Cu") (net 1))
 (segment (start 37.7569 21.4512) (end 36.8289 20.5232) (width 0.381) (layer "F.Cu") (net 1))
 (segment (start 37.7569 21.752774) (end 37.7569 22.9999) (width 0.381) (layer "F.Cu") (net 1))
 (segment (start 37.6188 23.992799) (end 38.767151 25.141149) (width 0.381) (layer "F.Cu") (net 1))
 (segment (start 39.198951 25.141149) (end 39.4716 24.8685) (width 0.381) (layer "F.Cu") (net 1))
 (segment (start 39.3465 15.3924) (end 37.0059 15.3924) (width 0.1524) (layer "F.Cu") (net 4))
 (segment (start 40.535599 22.064201) (end 40.535599 23.904201) (width 0.1524) (layer "F.Cu") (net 4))
 (segment (start 37.6428 20.677086) (end 38.227 21.261286) (width 0.1524) (layer "F.Cu") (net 4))
 (segment (start 37.0059 15.3924) (end 36.9551 15.4432) (width 0.1524) (layer "F.Cu") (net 4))
 (segment (start 37.6428 18.345918) (end 37.6428 20.677086) (width 0.1524) (layer "F.Cu") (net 4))
 (segment (start 38.227 21.8948) (end 38.272601 21.940401) (width 0.1524) (layer "F.Cu") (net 4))
 (segment (start 40.3714 24.0684) (end 40.535599 23.904201) (width 0.1524) (layer "F.Cu") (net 4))
 (segment (start 38.272601 21.940401) (end 39.522799 21.940401) (width 0.1524) (layer "F.Cu") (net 4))
 (segment (start 41.9845 25.6322) (end 40.672318 25.6322) (width 0.1524) (layer "F.Cu") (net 4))
 (segment (start 36.066 17.4986) (end 36.6122 18.0448) (width 0.1524) (layer "F.Cu") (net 4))
 (segment (start 36.6122 18.0448) (end 37.341682 18.0448) (width 0.1524) (layer "F.Cu") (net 4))
 (segment (start 36.066 16.3323) (end 36.066 17.4986) (width 0.1524) (layer "F.Cu") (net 4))
 (segment (start 38.227 21.261286) (end 38.227 21.8948) (width 0.1524) (layer "F.Cu") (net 4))
 (segment (start 40.411799 21.940401) (end 40.535599 22.064201) (width 0.1524) (layer "F.Cu") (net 4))
 (segment (start 42.7482 24.8685) (end 41.9845 25.6322) (width 0.1524) (layer "F.Cu") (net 4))
 (segment (start 39.522799 21.940401) (end 40.411799 21.940401) (width 0.1524) (layer "F.Cu") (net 4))
 (segment (start 40.672318 25.6322) (end 40.3714 25.331282) (width 0.1524) (layer "F.Cu") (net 4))
 (segment (start 36.9551 15.4432) (end 36.066 16.3323) (width 0.1524) (layer "F.Cu") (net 4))
 (segment (start 37.341682 18.0448) (end 37.6428 18.345918) (width 0.1524) (layer "F.Cu") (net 4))
 (segment (start 40.3714 25.331282) (end 40.3714 24.0684) (width 0.1524) (layer "F.Cu") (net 4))
 (segment (start 39.326801 21.094401) (end 39.522799 21.290399) (width 0.1524) (layer "F.Cu") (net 11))
 (segment (start 36.8797 17.0434) (end 37.8714 17.0434) (width 0.1524) (layer "F.Cu") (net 11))
 (segment (start 38.1508 17.0434) (end 39.2449 17.0434) (width 0.1524) (layer "F.Cu") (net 11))
 (segment (start 39.2449 17.0434) (end 39.2957 17.0942) (width 0.1524) (layer "F.Cu") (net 11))
 (segment (start 38.558484 21.094401) (end 37.9952 20.531117) (width 0.1524) (layer "F.Cu") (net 11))
 (segment (start 37.8714 17.0434) (end 38.1508 17.0434) (width 0.1524) (layer "F.Cu") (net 11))
 (segment (start 37.9952 20.531117) (end 37.9952 17.1672) (width 0.1524) (layer "F.Cu") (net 11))
 (segment (start 38.558484 21.094401) (end 39.326801 21.094401) (width 0.1524) (layer "F.Cu") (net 11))
 (segment (start 37.9952 17.1672) (end 37.8714 17.0434) (width 0.1524) (layer "F.Cu") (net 11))
 (segment (start 40.3117 17.7546) (end 39.2957 18.7706) (width 0.1524) (layer "F.Cu") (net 10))
 (segment (start 40.3117 16.2522) (end 40.3117 17.7546) (width 0.1524) (layer "F.Cu") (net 10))
 (segment (start 39.522799 18.997699) (end 39.522799 20.640401) (width 0.1524) (layer "F.Cu") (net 10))
 (segment (start 41.1715 15.3924) (end 40.3117 16.2522) (width 0.1524) (layer "F.Cu") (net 10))
 (segment (start 39.2957 18.7706) (end 39.522799 18.997699) (width 0.1524) (layer "F.Cu") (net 10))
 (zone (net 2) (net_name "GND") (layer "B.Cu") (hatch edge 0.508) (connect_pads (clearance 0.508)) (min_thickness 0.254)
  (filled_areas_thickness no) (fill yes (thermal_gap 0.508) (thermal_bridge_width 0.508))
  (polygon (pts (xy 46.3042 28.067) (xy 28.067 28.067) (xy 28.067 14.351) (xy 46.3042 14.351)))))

